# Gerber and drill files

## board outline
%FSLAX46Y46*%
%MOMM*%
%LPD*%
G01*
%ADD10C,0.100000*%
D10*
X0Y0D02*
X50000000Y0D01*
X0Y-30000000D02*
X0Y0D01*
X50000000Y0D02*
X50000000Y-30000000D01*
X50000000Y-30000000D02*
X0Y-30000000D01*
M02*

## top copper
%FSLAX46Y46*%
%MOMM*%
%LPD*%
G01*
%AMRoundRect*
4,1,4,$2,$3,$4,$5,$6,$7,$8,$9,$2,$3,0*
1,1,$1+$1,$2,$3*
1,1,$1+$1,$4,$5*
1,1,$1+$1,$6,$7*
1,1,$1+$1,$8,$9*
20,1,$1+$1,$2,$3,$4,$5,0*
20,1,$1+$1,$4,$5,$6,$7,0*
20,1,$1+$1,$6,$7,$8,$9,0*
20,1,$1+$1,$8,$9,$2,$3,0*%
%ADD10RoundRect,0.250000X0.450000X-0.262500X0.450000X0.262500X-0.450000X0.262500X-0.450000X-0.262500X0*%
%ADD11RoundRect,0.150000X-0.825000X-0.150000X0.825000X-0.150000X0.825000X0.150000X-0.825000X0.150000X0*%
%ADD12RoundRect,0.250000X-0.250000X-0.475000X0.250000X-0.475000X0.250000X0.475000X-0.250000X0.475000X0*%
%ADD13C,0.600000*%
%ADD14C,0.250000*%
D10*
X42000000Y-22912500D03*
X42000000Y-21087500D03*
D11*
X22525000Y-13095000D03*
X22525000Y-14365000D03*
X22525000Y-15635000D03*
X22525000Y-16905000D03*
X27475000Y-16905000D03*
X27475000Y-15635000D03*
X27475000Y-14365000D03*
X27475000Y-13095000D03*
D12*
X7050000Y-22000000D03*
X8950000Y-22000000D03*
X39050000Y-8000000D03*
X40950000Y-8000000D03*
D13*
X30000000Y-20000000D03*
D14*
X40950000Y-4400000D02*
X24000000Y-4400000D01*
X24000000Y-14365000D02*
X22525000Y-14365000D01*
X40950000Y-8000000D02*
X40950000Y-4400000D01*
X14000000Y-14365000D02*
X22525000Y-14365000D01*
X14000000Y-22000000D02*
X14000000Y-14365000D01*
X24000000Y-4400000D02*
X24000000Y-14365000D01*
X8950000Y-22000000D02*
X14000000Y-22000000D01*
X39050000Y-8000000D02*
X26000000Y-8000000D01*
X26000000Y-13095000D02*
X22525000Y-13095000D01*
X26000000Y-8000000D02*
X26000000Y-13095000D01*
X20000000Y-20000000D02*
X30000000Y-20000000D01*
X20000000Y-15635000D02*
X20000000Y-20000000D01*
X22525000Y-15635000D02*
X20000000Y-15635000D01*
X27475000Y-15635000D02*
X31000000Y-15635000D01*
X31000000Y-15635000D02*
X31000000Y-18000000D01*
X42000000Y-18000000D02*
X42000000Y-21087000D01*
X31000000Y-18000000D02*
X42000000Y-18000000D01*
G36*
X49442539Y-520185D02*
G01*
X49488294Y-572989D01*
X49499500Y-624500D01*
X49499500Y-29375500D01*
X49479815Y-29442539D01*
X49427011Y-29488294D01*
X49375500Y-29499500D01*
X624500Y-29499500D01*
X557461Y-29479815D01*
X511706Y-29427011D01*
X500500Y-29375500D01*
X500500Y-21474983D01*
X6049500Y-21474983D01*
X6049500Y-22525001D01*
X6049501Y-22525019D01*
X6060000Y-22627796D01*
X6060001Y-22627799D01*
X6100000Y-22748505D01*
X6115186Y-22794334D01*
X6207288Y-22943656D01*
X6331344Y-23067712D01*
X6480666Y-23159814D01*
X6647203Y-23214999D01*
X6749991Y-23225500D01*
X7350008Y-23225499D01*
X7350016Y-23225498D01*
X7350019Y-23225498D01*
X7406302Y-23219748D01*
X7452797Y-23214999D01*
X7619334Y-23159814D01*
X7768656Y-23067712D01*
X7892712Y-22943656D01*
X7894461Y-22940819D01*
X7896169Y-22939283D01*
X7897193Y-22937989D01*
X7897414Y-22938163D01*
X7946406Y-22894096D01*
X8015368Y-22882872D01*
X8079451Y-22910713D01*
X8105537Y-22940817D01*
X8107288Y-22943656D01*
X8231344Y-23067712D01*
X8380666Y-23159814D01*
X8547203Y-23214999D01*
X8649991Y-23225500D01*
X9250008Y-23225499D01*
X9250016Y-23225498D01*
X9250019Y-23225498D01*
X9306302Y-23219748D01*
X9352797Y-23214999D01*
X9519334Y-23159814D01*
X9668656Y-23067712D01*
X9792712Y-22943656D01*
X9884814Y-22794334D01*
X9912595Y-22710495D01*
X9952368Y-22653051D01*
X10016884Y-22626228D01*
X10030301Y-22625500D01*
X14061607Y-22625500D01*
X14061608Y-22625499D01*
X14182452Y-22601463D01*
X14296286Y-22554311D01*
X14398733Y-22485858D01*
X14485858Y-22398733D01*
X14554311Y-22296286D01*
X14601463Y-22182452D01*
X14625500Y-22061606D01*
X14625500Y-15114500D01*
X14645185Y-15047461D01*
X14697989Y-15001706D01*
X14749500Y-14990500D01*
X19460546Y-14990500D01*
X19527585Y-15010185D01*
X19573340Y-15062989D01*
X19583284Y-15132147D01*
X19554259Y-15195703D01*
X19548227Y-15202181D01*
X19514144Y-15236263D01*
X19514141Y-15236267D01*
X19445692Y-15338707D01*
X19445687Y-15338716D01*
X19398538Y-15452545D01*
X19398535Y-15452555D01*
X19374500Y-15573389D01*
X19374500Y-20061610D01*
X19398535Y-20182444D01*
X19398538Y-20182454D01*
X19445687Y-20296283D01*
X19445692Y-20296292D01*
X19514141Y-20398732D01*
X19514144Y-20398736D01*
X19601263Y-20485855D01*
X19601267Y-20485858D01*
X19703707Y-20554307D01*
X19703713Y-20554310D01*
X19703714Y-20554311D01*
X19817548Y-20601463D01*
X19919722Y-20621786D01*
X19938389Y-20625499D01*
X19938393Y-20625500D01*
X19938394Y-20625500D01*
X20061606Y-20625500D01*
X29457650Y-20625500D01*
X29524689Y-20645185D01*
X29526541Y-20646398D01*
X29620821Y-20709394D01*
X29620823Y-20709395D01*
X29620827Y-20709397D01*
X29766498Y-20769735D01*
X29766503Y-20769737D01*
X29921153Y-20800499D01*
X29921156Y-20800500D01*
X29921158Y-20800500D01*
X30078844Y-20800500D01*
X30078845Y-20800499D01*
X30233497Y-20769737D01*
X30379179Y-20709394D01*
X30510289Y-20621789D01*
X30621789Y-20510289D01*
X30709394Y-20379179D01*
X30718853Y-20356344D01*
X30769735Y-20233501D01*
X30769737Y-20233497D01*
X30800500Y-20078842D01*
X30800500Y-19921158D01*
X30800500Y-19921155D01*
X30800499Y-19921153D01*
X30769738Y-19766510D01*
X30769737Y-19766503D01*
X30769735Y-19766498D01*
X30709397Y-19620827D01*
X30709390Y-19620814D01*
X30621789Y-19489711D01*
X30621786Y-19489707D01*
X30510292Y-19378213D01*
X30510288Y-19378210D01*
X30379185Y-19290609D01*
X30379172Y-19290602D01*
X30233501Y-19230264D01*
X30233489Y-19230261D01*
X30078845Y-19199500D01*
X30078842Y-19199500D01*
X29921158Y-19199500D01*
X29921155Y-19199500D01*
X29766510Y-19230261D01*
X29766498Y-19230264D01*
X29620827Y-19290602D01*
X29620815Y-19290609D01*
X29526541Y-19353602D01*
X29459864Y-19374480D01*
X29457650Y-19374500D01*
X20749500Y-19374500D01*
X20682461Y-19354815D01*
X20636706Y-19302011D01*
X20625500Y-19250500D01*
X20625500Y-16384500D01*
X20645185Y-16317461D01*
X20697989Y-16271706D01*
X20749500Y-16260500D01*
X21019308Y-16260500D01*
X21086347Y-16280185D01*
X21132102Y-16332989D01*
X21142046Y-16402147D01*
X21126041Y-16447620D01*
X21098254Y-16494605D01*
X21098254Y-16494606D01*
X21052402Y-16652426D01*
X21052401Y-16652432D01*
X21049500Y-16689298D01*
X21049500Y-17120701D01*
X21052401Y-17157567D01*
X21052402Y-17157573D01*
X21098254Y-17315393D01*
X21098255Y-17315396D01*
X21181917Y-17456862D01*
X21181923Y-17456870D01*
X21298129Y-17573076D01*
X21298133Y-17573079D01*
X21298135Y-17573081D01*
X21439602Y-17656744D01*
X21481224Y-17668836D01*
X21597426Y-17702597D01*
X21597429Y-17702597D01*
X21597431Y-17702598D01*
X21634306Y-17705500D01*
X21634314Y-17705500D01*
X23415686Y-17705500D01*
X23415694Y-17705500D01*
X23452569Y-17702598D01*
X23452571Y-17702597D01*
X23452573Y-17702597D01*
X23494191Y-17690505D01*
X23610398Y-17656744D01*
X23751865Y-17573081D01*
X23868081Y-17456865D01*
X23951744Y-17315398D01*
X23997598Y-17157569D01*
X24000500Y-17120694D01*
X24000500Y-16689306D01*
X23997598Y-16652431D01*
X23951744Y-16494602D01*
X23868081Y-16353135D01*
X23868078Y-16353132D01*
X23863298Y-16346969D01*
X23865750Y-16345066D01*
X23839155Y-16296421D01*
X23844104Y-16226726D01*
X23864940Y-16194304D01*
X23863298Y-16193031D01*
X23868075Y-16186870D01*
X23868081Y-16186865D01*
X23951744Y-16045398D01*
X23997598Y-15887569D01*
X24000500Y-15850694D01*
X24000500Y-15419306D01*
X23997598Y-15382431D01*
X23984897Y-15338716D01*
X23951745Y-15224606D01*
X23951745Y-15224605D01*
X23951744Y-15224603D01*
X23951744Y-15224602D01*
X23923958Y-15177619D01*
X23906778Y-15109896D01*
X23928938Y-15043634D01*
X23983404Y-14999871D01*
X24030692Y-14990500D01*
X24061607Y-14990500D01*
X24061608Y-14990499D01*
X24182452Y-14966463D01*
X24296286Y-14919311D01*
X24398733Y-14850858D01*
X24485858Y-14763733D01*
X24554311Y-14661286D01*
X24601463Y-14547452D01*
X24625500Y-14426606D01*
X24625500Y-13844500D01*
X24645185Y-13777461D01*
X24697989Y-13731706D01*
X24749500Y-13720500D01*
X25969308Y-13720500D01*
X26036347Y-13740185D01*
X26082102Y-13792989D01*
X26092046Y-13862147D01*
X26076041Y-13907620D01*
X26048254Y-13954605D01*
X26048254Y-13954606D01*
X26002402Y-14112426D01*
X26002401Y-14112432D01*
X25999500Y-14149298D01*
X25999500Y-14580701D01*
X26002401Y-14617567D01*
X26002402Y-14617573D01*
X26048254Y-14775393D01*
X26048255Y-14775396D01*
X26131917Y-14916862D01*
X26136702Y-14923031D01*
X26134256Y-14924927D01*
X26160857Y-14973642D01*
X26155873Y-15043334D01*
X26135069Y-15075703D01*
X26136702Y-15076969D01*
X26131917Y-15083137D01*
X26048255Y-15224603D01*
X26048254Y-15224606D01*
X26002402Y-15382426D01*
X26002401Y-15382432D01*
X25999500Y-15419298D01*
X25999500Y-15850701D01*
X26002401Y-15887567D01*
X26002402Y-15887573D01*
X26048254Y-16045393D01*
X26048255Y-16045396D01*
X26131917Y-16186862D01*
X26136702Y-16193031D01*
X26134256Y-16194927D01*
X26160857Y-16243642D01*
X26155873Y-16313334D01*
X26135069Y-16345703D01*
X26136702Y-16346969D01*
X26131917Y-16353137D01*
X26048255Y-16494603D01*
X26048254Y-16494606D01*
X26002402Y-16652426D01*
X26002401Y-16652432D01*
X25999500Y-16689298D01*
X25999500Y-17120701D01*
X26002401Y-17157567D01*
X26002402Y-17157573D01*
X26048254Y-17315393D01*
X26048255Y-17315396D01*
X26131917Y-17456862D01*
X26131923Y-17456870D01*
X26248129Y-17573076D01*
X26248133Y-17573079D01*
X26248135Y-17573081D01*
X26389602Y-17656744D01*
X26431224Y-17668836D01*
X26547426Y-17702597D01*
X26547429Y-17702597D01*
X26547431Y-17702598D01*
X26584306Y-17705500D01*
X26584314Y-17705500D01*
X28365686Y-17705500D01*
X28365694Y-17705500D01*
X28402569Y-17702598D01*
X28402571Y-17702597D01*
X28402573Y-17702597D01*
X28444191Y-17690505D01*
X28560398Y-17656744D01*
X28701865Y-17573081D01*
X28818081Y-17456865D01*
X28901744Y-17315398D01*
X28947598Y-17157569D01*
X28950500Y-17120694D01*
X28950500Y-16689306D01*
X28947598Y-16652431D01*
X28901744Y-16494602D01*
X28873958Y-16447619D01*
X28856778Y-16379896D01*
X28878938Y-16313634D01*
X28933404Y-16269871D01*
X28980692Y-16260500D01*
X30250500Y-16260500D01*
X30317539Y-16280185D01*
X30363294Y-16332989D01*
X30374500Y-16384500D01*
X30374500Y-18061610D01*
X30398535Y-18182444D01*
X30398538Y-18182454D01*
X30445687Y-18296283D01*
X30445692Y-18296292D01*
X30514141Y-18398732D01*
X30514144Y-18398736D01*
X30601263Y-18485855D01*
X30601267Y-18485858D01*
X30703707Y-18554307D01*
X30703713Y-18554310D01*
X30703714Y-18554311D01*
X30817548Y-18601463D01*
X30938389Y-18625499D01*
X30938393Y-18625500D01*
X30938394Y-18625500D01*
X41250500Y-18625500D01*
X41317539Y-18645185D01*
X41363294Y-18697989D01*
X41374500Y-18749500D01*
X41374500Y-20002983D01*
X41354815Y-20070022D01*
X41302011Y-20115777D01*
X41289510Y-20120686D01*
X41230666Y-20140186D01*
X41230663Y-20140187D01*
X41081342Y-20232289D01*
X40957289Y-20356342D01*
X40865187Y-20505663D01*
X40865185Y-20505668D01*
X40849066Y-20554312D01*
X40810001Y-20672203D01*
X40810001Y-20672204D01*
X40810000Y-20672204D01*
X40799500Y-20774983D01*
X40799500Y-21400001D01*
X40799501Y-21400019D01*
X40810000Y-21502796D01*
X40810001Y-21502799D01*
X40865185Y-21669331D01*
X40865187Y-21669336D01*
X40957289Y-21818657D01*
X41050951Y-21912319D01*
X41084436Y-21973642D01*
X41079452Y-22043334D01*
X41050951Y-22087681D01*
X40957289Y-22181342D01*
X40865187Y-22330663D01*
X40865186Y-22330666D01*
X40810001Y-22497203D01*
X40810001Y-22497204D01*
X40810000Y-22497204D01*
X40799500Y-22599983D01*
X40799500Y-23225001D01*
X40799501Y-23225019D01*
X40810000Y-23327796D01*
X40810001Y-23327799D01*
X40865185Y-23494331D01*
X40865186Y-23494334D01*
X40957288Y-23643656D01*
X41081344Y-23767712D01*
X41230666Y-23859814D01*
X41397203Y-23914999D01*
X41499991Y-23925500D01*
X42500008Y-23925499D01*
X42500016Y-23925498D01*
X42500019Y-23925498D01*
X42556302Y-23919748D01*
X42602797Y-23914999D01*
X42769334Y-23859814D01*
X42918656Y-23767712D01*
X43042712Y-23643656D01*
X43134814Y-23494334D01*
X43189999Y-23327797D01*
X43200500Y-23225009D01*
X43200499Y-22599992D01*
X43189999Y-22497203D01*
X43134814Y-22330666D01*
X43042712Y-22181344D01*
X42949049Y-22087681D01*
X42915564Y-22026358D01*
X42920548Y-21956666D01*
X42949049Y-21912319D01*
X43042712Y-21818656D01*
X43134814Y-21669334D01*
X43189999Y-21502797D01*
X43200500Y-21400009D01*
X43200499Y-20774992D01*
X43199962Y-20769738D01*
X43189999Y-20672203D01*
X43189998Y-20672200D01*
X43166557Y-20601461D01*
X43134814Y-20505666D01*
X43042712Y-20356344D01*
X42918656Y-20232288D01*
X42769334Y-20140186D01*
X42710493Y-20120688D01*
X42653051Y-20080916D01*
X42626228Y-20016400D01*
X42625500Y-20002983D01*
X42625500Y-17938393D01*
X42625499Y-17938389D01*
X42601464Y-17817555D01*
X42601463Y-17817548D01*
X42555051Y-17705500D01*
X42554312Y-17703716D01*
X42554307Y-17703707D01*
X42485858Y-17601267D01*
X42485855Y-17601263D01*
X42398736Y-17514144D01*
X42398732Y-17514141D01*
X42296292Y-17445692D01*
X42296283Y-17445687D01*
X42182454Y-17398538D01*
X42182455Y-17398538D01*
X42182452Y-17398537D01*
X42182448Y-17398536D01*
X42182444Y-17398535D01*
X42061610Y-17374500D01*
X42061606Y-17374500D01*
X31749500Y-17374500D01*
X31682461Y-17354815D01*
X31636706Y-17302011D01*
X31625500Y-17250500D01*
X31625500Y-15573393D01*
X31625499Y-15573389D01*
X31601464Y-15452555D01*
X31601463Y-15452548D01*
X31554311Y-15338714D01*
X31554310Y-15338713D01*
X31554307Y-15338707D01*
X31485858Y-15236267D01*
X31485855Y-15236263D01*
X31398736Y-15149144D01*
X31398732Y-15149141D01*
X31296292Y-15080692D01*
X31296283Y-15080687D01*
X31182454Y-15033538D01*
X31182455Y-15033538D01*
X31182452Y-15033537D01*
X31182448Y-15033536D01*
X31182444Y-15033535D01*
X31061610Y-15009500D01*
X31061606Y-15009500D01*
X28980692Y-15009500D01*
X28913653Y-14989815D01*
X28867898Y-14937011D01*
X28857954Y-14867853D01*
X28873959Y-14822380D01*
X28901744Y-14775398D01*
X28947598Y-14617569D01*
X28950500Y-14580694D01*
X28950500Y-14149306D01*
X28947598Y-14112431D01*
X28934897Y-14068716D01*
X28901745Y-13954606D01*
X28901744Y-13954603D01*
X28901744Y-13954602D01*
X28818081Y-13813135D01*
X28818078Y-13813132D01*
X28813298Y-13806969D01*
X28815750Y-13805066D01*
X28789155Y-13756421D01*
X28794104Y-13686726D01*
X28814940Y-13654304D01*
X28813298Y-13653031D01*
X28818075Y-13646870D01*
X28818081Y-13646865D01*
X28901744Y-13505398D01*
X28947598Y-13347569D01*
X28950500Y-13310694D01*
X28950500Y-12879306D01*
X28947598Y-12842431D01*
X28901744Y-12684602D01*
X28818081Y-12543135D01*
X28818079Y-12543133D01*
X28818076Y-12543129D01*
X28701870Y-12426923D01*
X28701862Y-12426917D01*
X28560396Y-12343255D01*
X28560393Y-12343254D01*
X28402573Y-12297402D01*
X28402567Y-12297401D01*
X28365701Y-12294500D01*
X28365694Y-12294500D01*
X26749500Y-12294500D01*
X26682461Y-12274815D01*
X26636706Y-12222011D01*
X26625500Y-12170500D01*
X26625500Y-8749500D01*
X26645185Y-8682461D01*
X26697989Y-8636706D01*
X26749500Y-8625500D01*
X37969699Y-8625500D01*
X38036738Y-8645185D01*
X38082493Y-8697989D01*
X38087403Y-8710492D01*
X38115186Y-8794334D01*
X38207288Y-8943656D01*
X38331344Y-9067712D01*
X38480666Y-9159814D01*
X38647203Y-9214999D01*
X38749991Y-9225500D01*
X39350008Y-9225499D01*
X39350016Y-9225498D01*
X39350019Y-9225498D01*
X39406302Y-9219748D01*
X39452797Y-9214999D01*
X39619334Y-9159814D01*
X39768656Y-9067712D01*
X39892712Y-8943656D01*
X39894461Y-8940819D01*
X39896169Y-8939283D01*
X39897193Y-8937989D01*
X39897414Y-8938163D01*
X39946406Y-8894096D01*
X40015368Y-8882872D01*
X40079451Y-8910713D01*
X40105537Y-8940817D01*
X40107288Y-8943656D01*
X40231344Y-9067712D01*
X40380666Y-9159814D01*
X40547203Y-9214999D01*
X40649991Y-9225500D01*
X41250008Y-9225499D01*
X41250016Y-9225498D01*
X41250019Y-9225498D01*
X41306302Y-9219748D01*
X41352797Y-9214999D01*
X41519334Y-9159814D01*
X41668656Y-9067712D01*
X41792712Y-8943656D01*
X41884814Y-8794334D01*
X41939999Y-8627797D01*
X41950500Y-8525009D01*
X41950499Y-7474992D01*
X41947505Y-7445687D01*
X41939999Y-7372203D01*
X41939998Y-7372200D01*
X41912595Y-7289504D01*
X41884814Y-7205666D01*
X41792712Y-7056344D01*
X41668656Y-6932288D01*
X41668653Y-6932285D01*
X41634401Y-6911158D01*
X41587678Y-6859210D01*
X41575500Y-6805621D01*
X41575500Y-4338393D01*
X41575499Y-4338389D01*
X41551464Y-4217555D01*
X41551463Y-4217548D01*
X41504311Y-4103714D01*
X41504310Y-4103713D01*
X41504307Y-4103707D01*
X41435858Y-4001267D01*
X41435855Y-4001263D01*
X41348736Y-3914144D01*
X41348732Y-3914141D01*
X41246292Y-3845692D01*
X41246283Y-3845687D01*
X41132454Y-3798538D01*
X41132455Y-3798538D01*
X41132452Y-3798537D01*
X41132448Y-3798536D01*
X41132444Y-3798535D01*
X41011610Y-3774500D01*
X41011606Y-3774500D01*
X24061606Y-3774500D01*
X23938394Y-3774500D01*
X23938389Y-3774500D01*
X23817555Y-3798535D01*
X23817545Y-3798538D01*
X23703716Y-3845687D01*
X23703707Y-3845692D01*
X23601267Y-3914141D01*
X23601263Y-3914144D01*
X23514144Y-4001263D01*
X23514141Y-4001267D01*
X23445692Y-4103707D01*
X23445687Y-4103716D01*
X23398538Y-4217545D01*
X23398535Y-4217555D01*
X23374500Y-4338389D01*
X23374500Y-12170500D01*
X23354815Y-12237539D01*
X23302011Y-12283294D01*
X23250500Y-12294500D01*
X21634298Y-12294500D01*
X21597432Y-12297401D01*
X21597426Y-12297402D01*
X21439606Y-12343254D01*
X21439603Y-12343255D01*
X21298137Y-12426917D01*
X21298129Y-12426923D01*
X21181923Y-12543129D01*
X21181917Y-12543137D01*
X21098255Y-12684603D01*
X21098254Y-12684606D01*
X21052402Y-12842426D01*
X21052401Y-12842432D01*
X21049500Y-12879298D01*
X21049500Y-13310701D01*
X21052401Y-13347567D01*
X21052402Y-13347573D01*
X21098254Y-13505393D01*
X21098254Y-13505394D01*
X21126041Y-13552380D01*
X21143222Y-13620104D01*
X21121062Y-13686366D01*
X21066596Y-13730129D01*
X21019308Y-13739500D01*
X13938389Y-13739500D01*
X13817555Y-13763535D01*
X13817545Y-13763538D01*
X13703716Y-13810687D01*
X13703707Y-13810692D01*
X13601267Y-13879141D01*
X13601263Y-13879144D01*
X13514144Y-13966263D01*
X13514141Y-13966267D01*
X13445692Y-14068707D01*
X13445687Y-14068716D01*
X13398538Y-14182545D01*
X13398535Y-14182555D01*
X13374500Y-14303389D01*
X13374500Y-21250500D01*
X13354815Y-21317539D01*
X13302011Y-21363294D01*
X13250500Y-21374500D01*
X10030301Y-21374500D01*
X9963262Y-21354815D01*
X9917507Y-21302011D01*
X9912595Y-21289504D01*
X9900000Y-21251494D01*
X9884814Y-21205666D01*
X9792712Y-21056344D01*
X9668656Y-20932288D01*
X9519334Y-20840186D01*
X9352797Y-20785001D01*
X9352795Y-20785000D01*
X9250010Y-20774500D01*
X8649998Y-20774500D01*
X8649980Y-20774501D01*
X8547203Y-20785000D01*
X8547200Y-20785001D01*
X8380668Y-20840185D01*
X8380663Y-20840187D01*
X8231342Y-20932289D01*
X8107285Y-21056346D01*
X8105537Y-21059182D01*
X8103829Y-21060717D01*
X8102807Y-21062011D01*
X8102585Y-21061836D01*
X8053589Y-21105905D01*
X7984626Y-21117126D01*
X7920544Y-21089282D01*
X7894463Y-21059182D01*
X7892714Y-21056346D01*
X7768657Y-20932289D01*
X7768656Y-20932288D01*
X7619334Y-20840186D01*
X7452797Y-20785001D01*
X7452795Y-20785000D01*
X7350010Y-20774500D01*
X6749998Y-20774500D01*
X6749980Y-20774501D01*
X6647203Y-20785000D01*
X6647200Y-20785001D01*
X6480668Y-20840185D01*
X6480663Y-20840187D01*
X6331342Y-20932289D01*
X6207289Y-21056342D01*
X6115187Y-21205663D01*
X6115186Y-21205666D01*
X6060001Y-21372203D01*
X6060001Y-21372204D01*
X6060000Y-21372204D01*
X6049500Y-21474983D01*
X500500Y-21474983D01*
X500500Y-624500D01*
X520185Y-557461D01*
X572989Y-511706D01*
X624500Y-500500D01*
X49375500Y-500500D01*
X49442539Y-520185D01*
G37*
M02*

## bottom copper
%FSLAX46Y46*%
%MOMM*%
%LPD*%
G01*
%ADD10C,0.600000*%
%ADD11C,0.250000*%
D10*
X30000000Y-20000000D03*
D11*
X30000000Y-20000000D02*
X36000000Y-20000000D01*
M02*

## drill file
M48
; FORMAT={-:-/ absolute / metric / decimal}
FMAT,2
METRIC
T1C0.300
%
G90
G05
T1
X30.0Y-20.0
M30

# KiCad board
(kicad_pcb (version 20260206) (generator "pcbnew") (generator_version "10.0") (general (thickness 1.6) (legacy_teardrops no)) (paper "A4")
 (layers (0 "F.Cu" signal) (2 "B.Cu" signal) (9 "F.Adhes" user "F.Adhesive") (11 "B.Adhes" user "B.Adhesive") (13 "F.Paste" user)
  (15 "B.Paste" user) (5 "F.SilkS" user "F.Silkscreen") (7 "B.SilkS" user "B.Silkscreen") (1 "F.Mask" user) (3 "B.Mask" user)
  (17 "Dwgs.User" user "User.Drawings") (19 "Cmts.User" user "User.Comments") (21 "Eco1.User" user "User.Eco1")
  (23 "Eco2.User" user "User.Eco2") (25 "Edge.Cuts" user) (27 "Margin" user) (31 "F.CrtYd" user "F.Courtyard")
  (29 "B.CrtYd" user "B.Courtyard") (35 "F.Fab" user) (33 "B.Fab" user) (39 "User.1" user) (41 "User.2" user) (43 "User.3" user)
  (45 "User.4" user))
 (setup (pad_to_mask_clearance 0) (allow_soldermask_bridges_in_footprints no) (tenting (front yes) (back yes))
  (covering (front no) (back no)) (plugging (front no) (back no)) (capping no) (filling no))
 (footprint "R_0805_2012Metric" (layer "F.Cu") (at 42 22 90)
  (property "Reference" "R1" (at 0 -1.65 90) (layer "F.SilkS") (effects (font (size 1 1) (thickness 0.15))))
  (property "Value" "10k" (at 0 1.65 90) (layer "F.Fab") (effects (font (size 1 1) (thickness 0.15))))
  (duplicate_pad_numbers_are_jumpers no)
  (pad "1" smd roundrect (at -0.9125 0 90) (size 1.025 1.4) (layers "F.Cu" "F.Mask" "F.Paste") (roundrect_rratio 0.243902))
  (pad "2" smd roundrect (at 0.9125 0 90) (size 1.025 1.4) (layers "F.Cu" "F.Mask" "F.Paste") (roundrect_rratio 0.243902) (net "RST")))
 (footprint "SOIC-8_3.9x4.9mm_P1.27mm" (layer "F.Cu") (at 25 15)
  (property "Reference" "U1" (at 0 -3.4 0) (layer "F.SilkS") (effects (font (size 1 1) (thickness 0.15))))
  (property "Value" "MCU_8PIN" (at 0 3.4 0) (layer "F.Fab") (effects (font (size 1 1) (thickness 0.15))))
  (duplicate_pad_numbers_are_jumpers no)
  (pad "1" smd roundrect (at -2.475 -1.905) (size 1.95 0.6) (layers "F.Cu" "F.Mask" "F.Paste") (roundrect_rratio 0.25) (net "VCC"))
  (pad "2" smd roundrect (at -2.475 -0.635) (size 1.95 0.6) (layers "F.Cu" "F.Mask" "F.Paste") (roundrect_rratio 0.25) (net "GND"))
  (pad "3" smd roundrect (at -2.475 0.635) (size 1.95 0.6) (layers "F.Cu" "F.Mask" "F.Paste") (roundrect_rratio 0.25) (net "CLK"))
  (pad "4" smd roundrect (at -2.475 1.905) (size 1.95 0.6) (layers "F.Cu" "F.Mask" "F.Paste") (roundrect_rratio 0.25) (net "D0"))
  (pad "5" smd roundrect (at 2.475 1.905) (size 1.95 0.6) (layers "F.Cu" "F.Mask" "F.Paste") (roundrect_rratio 0.25) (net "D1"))
  (pad "6" smd roundrect (at 2.475 0.635) (size 1.95 0.6) (layers "F.Cu" "F.Mask" "F.Paste") (roundrect_rratio 0.25) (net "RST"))
  (pad "7" smd roundrect (at 2.475 -0.635) (size 1.95 0.6) (layers "F.Cu" "F.Mask" "F.Paste") (roundrect_rratio 0.25))
  (pad "8" smd roundrect (at 2.475 -1.905) (size 1.95 0.6) (layers "F.Cu" "F.Mask" "F.Paste") (roundrect_rratio 0.25)))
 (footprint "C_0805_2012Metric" (layer "F.Cu") (at 8 22)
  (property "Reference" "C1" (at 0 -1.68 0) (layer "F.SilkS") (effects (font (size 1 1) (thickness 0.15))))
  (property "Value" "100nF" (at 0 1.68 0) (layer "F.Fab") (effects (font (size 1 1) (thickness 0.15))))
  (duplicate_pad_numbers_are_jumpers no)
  (pad "1" smd roundrect (at -0.95 0) (size 1 1.45) (layers "F.Cu" "F.Mask" "F.Paste") (roundrect_rratio 0.25))
  (pad "2" smd roundrect (at 0.95 0) (size 1 1.45) (layers "F.Cu" "F.Mask" "F.Paste") (roundrect_rratio 0.25) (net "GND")))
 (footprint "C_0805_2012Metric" (layer "F.Cu") (at 40 8)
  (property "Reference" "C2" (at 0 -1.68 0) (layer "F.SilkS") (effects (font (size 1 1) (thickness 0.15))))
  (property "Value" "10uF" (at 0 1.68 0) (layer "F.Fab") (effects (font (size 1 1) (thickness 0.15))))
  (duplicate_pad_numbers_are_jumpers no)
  (pad "1" smd roundrect (at -0.95 0) (size 1 1.45) (layers "F.Cu" "F.Mask" "F.Paste") (roundrect_rratio 0.25) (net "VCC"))
  (pad "2" smd roundrect (at 0.95 0) (size 1 1.45) (layers "F.Cu" "F.Mask" "F.Paste") (roundrect_rratio 0.25) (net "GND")))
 (gr_line (start 0 0) (end 50 0) (stroke (width 0.1) (type default)) (layer "Edge.Cuts"))
 (gr_line (start 0 30) (end 0 0) (stroke (width 0.1) (type default)) (layer "Edge.Cuts"))
 (gr_line (start 50 0) (end 50 30) (stroke (width 0.1) (type default)) (layer "Edge.Cuts"))
 (gr_line (start 50 30) (end 0 30) (stroke (width 0.1) (type default)) (layer "Edge.Cuts"))
 (segment (start 40.95 4.4) (end 24 4.4) (width 0.25) (layer "F.Cu") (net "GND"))
 (segment (start 24 14.365) (end 22.525 14.365) (width 0.25) (layer "F.Cu") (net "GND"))
 (segment (start 40.95 8) (end 40.95 4.4) (width 0.25) (layer "F.Cu") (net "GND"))
 (segment (start 14 14.365) (end 22.525 14.365) (width 0.25) (layer "F.Cu") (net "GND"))
 (segment (start 14 22) (end 14 14.365) (width 0.25) (layer "F.Cu") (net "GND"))
 (segment (start 24 4.4) (end 24 14.365) (width 0.25) (layer "F.Cu") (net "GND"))
 (segment (start 8.95 22) (end 14 22) (width 0.25) (layer "F.Cu") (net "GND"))
 (segment (start 39.05 8) (end 26 8) (width 0.25) (layer "F.Cu") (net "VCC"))
 (segment (start 26 13.095) (end 22.525 13.095) (width 0.25) (layer "F.Cu") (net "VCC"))
 (segment (start 26 8) (end 26 13.095) (width 0.25) (layer "F.Cu") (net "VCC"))
 (segment (start 20 20) (end 30 20) (width 0.25) (layer "F.Cu") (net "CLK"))
 (segment (start 20 15.635) (end 20 20) (width 0.25) (layer "F.Cu") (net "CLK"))
 (segment (start 22.525 15.635) (end 20 15.635) (width 0.25) (layer "F.Cu") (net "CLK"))
 (via (at 30 20) (size 0.6) (drill 0.3) (layers "F.Cu" "B.Cu") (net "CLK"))
 (segment (start 30 20) (end 36 20) (width 0.25) (layer "B.Cu") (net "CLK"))
 (segment (start 27.475 15.635) (end 31 15.635) (width 0.25) (layer "F.Cu") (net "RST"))
 (segment (start 31 15.635) (end 31 18) (width 0.25) (layer "F.Cu") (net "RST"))
 (segment (start 42 18) (end 42 21.087) (width 0.25) (layer "F.Cu") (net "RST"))
 (segment (start 31 18) (end 42 18) (width 0.25) (layer "F.Cu") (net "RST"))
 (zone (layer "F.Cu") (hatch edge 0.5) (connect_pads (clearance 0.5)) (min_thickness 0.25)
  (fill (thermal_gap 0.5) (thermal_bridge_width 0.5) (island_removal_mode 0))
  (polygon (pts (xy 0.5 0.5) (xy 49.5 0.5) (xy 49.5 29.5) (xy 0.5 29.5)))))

